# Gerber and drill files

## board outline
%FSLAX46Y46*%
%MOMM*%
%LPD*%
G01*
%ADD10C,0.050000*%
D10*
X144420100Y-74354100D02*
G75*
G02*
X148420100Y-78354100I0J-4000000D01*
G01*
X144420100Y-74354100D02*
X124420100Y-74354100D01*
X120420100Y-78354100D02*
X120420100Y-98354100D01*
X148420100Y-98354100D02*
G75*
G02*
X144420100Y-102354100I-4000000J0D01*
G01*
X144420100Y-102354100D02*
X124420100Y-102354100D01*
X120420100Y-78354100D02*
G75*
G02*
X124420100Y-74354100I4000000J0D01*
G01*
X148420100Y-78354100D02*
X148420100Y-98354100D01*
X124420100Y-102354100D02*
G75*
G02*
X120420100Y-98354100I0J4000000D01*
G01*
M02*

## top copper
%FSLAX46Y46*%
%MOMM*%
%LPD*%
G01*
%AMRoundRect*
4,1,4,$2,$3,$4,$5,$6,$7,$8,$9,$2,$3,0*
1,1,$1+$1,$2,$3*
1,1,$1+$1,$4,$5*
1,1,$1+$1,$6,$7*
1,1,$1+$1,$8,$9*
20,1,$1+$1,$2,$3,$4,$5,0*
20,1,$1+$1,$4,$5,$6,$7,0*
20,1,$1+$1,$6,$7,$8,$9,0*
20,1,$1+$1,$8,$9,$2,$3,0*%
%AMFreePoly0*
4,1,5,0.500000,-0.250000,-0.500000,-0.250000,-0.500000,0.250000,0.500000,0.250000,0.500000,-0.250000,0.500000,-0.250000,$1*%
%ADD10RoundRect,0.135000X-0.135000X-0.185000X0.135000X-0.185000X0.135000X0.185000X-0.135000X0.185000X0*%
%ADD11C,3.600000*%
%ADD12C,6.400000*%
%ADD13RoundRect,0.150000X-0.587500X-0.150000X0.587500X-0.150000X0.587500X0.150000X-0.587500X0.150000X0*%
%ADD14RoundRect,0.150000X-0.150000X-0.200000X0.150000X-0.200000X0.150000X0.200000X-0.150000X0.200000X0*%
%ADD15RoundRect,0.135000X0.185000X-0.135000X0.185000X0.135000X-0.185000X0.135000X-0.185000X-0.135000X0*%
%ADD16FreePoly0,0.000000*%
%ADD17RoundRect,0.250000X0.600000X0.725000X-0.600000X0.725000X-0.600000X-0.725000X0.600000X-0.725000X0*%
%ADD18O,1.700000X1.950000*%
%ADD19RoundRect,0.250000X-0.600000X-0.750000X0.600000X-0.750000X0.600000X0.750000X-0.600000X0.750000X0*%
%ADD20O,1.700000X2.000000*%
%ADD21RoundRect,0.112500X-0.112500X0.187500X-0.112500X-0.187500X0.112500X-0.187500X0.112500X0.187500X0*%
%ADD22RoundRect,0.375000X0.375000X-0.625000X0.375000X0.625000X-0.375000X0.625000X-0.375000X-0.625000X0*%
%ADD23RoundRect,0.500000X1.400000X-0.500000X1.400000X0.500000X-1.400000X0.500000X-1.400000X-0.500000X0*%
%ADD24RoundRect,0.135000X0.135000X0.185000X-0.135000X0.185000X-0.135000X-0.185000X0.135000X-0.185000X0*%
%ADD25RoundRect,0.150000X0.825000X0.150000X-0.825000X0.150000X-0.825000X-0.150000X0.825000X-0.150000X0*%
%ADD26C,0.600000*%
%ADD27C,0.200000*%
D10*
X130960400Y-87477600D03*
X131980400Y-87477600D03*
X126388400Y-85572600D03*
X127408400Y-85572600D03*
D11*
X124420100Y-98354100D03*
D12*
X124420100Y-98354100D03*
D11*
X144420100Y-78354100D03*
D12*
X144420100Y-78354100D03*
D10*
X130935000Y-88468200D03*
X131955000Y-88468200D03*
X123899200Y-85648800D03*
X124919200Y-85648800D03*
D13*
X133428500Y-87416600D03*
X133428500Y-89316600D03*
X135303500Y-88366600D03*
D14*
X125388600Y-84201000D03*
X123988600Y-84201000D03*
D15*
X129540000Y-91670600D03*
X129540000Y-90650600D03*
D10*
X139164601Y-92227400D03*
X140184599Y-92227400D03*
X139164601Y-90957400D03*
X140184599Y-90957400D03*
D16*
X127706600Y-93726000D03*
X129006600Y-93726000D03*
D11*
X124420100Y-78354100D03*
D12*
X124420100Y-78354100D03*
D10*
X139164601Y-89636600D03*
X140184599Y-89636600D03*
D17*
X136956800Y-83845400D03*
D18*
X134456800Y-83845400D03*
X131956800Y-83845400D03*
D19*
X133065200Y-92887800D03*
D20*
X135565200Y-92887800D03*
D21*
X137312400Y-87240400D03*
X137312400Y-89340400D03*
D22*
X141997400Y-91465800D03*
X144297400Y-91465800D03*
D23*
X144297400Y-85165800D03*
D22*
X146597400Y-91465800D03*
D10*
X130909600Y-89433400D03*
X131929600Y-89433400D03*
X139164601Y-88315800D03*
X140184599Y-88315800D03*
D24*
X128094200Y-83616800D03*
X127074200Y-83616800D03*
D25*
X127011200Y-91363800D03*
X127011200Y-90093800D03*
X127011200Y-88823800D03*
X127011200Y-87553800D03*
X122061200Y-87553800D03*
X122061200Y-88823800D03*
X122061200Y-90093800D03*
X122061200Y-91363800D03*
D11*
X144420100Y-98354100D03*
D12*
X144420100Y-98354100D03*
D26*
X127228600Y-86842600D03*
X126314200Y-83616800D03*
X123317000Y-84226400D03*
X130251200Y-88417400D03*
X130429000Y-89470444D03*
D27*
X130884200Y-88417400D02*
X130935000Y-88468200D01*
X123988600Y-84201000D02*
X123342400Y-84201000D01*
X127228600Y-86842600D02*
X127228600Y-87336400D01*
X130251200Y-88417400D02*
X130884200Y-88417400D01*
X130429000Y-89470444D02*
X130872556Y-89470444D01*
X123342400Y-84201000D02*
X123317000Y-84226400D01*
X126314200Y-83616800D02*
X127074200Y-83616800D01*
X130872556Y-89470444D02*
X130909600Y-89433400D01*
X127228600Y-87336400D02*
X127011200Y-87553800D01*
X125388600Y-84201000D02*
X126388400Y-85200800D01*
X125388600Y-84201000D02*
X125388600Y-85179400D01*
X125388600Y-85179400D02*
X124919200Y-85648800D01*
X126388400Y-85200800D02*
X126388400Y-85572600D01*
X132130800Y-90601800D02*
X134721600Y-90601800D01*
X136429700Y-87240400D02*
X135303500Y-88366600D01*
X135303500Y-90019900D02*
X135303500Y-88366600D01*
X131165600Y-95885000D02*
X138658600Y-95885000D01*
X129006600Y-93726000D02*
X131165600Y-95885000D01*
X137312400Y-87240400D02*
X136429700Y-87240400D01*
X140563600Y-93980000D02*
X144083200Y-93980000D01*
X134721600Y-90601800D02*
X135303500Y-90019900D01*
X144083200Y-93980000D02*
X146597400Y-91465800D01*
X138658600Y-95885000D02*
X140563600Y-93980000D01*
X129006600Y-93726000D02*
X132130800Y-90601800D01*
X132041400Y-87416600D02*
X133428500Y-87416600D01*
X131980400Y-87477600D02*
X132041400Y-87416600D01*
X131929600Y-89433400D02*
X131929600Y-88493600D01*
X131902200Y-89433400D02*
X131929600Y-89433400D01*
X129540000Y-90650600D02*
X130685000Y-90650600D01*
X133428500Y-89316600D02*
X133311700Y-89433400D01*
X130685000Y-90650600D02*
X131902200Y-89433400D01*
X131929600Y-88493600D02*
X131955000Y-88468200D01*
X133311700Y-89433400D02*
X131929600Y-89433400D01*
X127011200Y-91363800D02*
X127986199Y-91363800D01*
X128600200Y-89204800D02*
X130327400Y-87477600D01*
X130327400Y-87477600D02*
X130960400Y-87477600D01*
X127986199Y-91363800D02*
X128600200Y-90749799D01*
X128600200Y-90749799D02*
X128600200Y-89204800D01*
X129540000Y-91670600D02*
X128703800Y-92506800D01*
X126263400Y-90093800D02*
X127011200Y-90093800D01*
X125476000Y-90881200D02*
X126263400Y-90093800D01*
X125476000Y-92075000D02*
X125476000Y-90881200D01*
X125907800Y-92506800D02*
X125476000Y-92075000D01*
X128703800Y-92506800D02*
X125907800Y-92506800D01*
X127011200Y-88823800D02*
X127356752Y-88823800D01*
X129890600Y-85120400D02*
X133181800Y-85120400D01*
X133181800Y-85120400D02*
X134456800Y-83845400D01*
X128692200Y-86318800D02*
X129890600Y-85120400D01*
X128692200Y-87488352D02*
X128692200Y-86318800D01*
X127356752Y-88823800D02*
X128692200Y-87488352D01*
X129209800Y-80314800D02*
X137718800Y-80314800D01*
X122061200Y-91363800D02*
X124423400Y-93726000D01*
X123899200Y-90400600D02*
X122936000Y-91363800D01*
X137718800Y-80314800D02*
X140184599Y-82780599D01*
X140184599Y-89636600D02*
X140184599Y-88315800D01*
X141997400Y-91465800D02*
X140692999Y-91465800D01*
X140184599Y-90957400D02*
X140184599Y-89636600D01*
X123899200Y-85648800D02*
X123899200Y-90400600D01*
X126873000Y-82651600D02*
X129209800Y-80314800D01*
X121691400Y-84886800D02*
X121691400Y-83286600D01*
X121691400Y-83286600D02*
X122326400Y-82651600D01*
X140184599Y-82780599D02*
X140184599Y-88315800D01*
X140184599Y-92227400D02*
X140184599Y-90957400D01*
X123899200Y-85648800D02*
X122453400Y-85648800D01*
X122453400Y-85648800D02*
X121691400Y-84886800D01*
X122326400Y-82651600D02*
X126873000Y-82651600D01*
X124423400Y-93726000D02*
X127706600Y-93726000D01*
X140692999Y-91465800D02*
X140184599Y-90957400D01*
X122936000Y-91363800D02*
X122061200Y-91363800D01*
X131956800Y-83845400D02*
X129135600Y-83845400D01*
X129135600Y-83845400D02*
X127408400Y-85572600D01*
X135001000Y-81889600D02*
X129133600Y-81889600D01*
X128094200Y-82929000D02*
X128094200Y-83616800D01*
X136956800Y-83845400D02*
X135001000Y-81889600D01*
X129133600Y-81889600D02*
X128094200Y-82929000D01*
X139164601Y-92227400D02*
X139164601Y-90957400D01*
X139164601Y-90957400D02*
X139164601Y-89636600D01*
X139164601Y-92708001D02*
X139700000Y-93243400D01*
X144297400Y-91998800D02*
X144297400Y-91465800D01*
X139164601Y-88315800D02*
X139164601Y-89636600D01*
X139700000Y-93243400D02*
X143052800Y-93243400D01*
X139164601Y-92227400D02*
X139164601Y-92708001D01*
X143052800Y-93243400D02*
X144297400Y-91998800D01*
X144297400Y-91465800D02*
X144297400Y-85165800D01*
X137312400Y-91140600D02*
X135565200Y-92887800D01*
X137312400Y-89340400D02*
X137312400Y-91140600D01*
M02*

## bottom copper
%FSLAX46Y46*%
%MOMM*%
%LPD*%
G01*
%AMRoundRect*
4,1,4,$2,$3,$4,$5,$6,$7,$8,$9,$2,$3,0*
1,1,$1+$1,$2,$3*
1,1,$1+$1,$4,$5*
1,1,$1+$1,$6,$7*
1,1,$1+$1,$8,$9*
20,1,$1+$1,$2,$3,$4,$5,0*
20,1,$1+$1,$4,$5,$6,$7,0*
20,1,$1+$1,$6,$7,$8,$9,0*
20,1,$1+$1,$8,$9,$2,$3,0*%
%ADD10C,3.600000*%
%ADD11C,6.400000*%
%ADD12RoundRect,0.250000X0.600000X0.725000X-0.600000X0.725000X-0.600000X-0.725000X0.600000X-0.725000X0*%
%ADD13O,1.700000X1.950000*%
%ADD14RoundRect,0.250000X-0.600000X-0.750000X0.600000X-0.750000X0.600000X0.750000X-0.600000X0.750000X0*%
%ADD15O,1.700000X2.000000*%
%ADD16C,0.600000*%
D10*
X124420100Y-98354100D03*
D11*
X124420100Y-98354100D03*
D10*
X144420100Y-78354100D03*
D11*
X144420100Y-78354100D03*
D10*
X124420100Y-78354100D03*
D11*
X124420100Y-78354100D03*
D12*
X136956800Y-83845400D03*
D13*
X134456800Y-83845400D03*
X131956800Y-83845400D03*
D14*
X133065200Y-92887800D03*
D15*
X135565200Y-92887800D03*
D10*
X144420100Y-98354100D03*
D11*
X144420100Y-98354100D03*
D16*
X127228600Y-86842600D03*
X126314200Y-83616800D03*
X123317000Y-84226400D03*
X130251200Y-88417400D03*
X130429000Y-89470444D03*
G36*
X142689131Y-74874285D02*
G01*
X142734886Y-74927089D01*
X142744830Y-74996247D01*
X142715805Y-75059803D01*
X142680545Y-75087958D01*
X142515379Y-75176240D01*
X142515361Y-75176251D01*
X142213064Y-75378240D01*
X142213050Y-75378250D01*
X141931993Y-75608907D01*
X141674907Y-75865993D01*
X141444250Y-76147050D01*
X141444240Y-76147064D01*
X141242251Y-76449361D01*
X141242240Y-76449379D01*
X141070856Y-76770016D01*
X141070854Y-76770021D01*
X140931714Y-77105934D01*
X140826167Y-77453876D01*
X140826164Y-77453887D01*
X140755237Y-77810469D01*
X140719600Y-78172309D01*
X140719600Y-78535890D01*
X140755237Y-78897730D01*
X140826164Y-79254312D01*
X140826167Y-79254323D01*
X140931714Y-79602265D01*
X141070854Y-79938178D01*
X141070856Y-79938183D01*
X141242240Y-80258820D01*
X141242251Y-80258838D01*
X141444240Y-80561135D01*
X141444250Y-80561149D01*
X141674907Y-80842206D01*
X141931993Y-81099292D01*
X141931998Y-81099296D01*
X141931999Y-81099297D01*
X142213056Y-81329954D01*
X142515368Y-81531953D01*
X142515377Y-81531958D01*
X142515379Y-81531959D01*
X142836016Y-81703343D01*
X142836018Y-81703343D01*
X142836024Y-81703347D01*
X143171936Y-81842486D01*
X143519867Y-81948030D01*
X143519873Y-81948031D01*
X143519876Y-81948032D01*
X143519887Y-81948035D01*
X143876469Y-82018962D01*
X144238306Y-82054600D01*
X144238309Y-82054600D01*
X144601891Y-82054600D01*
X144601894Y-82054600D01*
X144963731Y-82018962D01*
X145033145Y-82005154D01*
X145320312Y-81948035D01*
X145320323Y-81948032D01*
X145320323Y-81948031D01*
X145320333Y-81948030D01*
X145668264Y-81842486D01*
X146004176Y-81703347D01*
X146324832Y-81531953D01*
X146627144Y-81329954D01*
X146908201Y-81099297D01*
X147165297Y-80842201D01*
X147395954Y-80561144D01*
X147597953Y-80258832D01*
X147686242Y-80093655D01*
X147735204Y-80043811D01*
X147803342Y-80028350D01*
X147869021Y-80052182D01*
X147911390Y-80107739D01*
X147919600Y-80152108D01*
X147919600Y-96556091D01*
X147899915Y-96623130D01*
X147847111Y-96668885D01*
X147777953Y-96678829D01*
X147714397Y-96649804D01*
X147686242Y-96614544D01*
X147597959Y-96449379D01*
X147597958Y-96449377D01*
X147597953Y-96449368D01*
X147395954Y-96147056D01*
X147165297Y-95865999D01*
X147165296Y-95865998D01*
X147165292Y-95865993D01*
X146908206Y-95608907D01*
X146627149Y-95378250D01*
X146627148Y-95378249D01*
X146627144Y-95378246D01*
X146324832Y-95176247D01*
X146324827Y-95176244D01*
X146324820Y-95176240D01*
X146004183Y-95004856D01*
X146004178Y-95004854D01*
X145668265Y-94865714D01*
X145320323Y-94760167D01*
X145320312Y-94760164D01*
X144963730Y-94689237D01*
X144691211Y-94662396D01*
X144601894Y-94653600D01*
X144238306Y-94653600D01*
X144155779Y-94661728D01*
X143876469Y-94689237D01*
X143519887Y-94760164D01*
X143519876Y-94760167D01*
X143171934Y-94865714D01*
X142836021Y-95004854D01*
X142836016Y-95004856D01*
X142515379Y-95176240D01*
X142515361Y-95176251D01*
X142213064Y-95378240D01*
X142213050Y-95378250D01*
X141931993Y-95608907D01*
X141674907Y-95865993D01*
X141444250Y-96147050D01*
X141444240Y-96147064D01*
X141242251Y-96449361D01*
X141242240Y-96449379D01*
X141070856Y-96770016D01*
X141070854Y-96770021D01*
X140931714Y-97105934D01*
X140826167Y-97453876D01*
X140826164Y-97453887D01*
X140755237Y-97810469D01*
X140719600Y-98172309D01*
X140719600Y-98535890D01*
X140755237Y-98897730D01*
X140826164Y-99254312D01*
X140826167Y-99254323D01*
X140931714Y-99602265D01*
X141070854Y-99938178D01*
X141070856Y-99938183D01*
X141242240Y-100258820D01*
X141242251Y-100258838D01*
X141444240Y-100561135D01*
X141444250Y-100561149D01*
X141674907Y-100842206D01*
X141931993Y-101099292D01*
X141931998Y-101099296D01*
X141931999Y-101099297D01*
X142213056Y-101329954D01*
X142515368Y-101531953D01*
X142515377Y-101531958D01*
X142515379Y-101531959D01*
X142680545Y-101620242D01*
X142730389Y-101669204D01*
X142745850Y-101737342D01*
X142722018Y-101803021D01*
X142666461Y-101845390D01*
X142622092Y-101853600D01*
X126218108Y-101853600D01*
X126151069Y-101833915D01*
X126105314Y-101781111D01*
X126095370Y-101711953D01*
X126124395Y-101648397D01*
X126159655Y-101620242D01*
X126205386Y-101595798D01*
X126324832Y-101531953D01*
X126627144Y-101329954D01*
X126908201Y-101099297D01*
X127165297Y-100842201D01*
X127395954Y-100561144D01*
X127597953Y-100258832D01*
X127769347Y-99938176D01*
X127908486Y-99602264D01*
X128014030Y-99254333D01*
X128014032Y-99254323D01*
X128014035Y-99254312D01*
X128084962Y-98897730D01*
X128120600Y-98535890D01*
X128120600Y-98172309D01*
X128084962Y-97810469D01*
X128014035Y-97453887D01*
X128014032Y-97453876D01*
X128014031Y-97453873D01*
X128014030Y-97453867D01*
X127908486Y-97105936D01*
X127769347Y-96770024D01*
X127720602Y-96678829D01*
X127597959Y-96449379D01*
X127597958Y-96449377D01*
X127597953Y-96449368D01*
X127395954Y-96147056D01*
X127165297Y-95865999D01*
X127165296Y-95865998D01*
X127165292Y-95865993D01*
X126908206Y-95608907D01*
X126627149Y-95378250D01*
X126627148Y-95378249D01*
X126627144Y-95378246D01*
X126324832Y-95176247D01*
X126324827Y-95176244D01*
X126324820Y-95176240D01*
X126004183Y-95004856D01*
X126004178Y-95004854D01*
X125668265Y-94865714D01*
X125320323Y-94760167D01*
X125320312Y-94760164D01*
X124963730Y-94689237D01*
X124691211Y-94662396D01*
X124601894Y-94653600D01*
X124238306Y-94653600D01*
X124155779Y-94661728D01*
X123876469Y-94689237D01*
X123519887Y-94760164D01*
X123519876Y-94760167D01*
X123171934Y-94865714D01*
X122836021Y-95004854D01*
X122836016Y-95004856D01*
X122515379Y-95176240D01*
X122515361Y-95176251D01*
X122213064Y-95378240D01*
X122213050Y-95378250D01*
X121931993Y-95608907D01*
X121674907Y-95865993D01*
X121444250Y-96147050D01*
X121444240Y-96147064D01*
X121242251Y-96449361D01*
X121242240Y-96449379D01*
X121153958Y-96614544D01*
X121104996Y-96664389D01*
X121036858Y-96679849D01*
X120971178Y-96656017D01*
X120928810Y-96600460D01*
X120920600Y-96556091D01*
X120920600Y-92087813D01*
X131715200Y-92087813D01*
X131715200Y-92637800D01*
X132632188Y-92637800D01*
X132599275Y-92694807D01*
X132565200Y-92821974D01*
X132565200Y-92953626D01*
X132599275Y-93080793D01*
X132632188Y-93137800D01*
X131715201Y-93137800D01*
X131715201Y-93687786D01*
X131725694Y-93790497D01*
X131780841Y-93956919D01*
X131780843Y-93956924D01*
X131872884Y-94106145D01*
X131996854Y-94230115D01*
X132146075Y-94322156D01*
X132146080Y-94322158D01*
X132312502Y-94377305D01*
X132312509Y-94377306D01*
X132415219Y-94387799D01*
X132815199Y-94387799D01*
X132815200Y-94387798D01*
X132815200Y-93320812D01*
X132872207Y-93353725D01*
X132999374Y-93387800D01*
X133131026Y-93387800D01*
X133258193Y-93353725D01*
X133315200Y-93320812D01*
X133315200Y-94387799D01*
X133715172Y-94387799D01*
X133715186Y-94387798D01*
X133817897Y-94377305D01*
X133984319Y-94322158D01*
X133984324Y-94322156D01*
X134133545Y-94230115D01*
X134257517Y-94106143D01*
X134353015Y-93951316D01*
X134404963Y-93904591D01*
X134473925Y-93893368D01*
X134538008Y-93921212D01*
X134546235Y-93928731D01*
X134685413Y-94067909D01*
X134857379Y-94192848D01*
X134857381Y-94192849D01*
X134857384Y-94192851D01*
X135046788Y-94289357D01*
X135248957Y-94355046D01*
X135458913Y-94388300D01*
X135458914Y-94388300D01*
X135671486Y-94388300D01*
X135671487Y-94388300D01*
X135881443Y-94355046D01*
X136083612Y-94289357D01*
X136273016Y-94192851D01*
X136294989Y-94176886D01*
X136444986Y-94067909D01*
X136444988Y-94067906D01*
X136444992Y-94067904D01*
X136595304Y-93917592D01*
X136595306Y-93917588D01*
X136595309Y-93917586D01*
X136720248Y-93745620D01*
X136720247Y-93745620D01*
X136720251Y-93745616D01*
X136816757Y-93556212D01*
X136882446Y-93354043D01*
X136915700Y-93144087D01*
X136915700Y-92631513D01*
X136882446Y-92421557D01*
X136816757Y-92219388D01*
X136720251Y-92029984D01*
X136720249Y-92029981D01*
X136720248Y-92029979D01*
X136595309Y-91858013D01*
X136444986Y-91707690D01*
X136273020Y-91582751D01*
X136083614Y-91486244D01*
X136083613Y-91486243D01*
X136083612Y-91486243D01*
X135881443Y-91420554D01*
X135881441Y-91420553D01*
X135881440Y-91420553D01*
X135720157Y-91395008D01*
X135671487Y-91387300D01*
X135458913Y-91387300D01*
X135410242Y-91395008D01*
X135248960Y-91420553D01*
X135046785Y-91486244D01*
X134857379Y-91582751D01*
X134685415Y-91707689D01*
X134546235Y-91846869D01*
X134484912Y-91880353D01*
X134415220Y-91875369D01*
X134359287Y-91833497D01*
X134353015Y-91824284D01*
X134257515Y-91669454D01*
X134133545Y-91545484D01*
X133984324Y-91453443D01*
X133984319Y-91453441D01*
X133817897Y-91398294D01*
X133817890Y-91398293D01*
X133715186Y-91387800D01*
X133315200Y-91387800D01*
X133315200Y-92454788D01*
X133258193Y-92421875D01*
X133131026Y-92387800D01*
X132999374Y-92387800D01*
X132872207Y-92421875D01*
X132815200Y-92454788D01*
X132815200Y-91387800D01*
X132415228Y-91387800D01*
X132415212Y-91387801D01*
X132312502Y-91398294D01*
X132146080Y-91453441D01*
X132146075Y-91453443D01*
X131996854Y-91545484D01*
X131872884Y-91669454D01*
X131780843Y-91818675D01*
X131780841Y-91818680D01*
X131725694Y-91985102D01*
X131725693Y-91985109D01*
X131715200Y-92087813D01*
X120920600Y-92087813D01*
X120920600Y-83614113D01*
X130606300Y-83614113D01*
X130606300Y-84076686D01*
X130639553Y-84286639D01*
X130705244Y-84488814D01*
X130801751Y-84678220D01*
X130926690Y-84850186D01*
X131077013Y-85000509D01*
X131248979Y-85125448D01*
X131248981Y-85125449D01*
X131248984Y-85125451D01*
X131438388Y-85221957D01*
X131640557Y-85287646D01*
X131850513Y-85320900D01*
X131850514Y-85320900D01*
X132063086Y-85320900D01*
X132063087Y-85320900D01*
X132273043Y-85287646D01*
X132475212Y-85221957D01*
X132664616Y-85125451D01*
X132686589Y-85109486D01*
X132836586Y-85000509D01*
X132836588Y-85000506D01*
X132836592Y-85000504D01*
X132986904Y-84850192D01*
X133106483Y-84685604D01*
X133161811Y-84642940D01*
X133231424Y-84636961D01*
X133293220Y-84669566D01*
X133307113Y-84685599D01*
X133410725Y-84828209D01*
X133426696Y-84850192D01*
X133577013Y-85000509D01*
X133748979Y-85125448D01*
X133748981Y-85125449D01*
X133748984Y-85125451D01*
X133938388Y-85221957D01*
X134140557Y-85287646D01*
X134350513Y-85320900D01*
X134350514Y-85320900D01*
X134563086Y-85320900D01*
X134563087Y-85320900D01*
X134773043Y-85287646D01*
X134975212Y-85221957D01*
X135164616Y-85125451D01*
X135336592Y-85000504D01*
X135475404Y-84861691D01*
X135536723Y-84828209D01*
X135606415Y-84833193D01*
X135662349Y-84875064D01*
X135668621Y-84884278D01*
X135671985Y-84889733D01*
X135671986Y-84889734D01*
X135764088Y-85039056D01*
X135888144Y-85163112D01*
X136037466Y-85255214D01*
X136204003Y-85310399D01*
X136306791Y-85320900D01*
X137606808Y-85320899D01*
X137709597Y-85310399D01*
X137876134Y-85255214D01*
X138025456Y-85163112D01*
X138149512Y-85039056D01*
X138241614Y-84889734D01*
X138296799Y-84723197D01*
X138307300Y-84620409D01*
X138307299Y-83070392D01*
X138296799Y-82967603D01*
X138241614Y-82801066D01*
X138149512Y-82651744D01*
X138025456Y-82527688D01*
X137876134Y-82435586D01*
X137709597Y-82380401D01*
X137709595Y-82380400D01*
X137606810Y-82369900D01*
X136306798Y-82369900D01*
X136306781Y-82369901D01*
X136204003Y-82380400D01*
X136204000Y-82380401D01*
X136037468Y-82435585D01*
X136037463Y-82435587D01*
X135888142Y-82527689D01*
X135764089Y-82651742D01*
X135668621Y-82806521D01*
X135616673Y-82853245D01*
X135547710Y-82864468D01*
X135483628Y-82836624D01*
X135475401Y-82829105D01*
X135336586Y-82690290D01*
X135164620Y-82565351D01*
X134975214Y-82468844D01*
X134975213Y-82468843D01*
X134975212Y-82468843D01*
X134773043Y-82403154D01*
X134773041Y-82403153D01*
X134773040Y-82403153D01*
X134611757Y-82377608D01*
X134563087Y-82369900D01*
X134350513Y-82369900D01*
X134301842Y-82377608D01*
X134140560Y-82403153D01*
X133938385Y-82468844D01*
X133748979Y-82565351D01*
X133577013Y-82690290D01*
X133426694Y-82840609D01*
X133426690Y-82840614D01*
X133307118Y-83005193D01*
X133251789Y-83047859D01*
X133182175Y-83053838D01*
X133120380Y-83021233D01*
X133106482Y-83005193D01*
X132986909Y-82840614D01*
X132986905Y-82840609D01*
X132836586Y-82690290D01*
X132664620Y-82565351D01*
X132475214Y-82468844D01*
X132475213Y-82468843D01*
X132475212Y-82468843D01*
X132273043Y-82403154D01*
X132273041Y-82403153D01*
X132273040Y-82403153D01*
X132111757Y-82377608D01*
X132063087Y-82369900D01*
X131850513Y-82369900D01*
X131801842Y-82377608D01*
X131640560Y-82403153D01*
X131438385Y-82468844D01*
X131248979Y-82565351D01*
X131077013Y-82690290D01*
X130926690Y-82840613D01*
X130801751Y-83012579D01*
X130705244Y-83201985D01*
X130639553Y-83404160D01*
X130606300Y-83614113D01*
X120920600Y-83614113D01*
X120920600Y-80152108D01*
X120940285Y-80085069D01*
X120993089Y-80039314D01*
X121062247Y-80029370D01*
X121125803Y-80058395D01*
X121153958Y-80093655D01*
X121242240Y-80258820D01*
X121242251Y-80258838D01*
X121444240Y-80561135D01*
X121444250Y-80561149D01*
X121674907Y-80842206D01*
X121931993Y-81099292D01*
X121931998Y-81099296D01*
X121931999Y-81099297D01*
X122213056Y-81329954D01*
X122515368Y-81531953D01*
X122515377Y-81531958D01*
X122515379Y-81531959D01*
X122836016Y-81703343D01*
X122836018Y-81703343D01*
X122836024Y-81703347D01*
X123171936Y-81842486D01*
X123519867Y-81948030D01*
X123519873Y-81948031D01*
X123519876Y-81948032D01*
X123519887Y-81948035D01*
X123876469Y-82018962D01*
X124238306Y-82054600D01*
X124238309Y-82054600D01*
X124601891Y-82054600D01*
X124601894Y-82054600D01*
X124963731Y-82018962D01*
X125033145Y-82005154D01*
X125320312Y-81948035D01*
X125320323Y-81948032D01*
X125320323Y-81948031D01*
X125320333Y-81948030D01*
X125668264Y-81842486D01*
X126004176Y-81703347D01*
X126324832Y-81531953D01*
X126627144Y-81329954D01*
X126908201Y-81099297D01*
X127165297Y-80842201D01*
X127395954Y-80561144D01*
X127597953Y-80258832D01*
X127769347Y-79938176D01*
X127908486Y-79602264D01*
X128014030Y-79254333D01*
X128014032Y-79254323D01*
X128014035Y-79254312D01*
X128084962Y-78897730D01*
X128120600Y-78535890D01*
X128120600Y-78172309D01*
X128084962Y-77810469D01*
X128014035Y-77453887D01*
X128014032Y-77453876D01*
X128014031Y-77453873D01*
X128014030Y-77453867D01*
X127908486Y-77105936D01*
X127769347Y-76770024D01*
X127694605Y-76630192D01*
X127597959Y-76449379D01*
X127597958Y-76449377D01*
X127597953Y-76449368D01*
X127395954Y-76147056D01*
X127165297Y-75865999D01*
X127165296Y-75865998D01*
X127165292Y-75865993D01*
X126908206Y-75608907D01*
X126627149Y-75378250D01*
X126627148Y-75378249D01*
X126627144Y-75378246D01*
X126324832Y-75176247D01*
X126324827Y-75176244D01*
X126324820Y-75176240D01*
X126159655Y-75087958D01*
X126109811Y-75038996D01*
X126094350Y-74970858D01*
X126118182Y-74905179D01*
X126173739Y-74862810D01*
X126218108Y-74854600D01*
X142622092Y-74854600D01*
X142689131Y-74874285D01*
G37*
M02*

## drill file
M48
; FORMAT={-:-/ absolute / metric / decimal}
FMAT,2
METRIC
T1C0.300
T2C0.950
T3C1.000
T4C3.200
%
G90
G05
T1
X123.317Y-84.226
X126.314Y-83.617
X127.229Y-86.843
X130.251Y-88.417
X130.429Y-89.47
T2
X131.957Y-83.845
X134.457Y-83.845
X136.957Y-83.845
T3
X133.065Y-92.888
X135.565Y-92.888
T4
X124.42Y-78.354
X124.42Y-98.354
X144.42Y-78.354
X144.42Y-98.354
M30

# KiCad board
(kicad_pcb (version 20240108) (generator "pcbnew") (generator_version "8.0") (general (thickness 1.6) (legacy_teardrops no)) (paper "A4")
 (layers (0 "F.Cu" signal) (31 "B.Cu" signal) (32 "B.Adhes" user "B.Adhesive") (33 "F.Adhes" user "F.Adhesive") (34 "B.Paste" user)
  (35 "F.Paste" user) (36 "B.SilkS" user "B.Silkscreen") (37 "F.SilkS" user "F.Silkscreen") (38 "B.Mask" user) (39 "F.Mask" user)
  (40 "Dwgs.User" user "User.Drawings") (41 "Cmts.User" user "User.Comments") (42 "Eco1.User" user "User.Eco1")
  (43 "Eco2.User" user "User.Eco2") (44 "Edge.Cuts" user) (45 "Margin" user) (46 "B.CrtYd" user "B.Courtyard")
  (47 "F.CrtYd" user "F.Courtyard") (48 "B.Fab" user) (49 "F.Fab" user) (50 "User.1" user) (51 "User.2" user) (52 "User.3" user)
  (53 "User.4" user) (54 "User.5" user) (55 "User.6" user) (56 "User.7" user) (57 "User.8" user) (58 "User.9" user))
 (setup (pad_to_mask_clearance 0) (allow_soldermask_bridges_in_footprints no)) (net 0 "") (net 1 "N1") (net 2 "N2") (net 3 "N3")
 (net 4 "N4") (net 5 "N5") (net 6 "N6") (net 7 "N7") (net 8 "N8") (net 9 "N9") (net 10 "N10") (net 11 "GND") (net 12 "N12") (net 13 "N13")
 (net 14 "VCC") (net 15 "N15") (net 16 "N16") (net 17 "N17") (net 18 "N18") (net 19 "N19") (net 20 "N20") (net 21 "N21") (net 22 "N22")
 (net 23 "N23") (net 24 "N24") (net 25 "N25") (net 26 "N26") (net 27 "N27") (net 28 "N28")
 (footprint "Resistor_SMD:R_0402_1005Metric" (layer "F.Cu") (at 131.4704 87.4776)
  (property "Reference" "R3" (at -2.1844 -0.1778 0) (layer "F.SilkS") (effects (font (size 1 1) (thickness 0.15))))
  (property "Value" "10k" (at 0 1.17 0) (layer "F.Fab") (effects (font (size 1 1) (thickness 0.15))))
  (pad "1" smd roundrect (at -0.51 0) (size 0.54 0.64) (layers "F.Cu" "F.Paste" "F.Mask") (roundrect_rratio 0.25) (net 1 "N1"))
  (pad "2" smd roundrect (at 0.51 0) (size 0.54 0.64) (layers "F.Cu" "F.Paste" "F.Mask") (roundrect_rratio 0.25) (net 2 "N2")))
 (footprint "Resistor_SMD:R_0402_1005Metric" (layer "F.Cu") (at 126.8984 85.5726)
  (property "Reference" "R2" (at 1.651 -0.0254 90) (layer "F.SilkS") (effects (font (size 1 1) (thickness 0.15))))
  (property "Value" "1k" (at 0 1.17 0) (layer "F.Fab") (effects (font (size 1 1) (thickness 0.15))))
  (pad "1" smd roundrect (at -0.51 0) (size 0.54 0.64) (layers "F.Cu" "F.Paste" "F.Mask") (roundrect_rratio 0.25) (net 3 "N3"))
  (pad "2" smd roundrect (at 0.51 0) (size 0.54 0.64) (layers "F.Cu" "F.Paste" "F.Mask") (roundrect_rratio 0.25) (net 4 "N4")))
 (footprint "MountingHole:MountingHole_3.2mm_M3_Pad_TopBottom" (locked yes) (layer "F.Cu") (at 124.4201 98.3541)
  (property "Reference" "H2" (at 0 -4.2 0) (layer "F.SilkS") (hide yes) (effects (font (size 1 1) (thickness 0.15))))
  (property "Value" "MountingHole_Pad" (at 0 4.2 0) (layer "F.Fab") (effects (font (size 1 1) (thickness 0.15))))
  (pad "1" thru_hole circle (at 0 0) (size 3.6 3.6) (drill 3.2) (layers "*.Cu" "*.Mask") (remove_unused_layers no) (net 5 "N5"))
  (pad "1" connect circle (at 0 0) (size 6.4 6.4) (layers "F.Cu" "F.Mask") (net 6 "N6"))
  (pad "1" connect circle (at 0 0) (size 6.4 6.4) (layers "B.Cu" "B.Mask") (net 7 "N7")))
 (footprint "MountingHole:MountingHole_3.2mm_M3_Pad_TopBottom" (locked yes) (layer "F.Cu") (at 144.4201 78.3541)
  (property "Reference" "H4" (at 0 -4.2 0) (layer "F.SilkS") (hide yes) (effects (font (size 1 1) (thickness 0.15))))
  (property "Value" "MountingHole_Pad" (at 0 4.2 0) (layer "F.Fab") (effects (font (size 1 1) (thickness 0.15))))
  (pad "1" thru_hole circle (at 0 0) (size 3.6 3.6) (drill 3.2) (layers "*.Cu" "*.Mask") (remove_unused_layers no) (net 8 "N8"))
  (pad "1" connect circle (at 0 0) (size 6.4 6.4) (layers "F.Cu" "F.Mask") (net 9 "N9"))
  (pad "1" connect circle (at 0 0) (size 6.4 6.4) (layers "B.Cu" "B.Mask") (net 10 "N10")))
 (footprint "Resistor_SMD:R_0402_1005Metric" (layer "F.Cu") (at 131.445 88.4682)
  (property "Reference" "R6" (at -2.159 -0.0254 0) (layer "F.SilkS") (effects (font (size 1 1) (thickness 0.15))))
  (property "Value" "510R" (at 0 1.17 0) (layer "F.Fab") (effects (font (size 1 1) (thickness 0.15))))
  (pad "1" smd roundrect (at -0.51 0) (size 0.54 0.64) (layers "F.Cu" "F.Paste" "F.Mask") (roundrect_rratio 0.25) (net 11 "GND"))
  (pad "2" smd roundrect (at 0.51 0) (size 0.54 0.64) (layers "F.Cu" "F.Paste" "F.Mask") (roundrect_rratio 0.25) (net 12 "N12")))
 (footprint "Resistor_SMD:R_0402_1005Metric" (layer "F.Cu") (at 124.4092 85.6488)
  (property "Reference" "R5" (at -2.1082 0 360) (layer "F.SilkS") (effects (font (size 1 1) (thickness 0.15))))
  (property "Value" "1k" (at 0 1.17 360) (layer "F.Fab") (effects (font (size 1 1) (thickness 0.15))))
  (pad "1" smd roundrect (at -0.51 0) (size 0.54 0.64) (layers "F.Cu" "F.Paste" "F.Mask") (roundrect_rratio 0.25) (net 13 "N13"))
  (pad "2" smd roundrect (at 0.51 0) (size 0.54 0.64) (layers "F.Cu" "F.Paste" "F.Mask") (roundrect_rratio 0.25) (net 3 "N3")))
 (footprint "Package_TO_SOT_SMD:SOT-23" (layer "F.Cu") (at 134.366 88.3666)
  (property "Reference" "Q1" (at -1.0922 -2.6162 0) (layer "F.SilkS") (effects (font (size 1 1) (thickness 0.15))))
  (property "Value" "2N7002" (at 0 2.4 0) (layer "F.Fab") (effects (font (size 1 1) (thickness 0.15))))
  (pad "1" smd roundrect (at -0.9375 -0.95) (size 1.475 0.6) (layers "F.Cu" "F.Paste" "F.Mask") (roundrect_rratio 0.25) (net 2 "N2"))
  (pad "2" smd roundrect (at -0.9375 0.95) (size 1.475 0.6) (layers "F.Cu" "F.Paste" "F.Mask") (roundrect_rratio 0.25) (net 12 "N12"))
  (pad "3" smd roundrect (at 0.9375 0) (size 1.475 0.6) (layers "F.Cu" "F.Paste" "F.Mask") (roundrect_rratio 0.25) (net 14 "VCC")))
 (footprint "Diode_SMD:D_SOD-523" (layer "F.Cu") (at 124.6886 84.201 180)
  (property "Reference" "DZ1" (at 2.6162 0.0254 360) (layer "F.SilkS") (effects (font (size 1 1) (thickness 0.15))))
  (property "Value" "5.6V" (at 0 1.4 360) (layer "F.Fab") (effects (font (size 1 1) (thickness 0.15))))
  (pad "1" smd roundrect (at -0.7 0) (size 0.6 0.7) (layers "F.Cu" "F.Paste" "F.Mask") (roundrect_rratio 0.25) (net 3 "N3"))
  (pad "2" smd roundrect (at 0.7 0) (size 0.6 0.7) (layers "F.Cu" "F.Paste" "F.Mask") (roundrect_rratio 0.25) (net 11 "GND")))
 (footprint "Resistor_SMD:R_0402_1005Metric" (layer "F.Cu") (at 129.54 91.1606 90)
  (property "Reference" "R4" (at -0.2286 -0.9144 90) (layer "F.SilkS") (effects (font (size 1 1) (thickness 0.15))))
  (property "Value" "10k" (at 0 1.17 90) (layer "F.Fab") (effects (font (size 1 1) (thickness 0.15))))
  (pad "1" smd roundrect (at -0.51 0 90) (size 0.54 0.64) (layers "F.Cu" "F.Paste" "F.Mask") (roundrect_rratio 0.25) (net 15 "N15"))
  (pad "2" smd roundrect (at 0.51 0 90) (size 0.54 0.64) (layers "F.Cu" "F.Paste" "F.Mask") (roundrect_rratio 0.25) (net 12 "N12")))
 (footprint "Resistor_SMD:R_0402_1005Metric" (layer "F.Cu") (at 139.6746 92.2274)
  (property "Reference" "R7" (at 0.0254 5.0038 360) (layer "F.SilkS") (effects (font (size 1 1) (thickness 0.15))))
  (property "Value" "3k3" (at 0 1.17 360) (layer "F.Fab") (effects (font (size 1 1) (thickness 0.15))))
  (pad "1" smd roundrect (at -0.509999 0) (size 0.54 0.64) (layers "F.Cu" "F.Paste" "F.Mask") (roundrect_rratio 0.25) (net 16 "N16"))
  (pad "2" smd roundrect (at 0.509999 0) (size 0.54 0.64) (layers "F.Cu" "F.Paste" "F.Mask") (roundrect_rratio 0.25) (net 13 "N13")))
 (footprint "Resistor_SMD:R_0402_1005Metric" (layer "F.Cu") (at 139.6746 90.9574)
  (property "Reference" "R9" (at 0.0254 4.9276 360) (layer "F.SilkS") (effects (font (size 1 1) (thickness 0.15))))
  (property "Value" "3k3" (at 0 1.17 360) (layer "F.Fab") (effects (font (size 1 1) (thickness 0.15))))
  (pad "1" smd roundrect (at -0.509999 0) (size 0.54 0.64) (layers "F.Cu" "F.Paste" "F.Mask") (roundrect_rratio 0.25) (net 16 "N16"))
  (pad "2" smd roundrect (at 0.509999 0) (size 0.54 0.64) (layers "F.Cu" "F.Paste" "F.Mask") (roundrect_rratio 0.25) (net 13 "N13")))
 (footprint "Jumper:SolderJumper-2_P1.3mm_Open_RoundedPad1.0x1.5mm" (layer "F.Cu") (at 128.3566 93.726)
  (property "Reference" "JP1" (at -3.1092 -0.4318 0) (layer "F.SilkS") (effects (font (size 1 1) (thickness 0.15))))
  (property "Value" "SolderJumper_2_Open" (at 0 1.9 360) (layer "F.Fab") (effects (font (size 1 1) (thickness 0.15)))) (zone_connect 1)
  (pad "1" smd custom (at -0.65 0) (size 1 0.5) (layers "F.Cu" "F.Mask") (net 13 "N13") (zone_connect 2) (thermal_bridge_angle 45)
   (options (clearance outline) (anchor rect)) (primitives))
  (pad "2" smd custom (at 0.65 0) (size 1 0.5) (layers "F.Cu" "F.Mask") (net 14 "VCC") (zone_connect 2) (thermal_bridge_angle 45)
   (options (clearance outline) (anchor rect)) (primitives)))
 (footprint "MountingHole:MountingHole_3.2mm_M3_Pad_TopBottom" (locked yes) (layer "F.Cu") (at 124.4201 78.3541)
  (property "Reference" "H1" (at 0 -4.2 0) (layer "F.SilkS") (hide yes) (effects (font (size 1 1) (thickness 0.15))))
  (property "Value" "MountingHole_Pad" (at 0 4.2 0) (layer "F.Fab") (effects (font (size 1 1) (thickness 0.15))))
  (pad "1" thru_hole circle (at 0 0) (size 3.6 3.6) (drill 3.2) (layers "*.Cu" "*.Mask") (remove_unused_layers no) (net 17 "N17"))
  (pad "1" connect circle (at 0 0) (size 6.4 6.4) (layers "F.Cu" "F.Mask") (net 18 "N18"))
  (pad "1" connect circle (at 0 0) (size 6.4 6.4) (layers "B.Cu" "B.Mask") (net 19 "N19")))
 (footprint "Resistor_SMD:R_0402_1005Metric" (layer "F.Cu") (at 139.6746 89.6366)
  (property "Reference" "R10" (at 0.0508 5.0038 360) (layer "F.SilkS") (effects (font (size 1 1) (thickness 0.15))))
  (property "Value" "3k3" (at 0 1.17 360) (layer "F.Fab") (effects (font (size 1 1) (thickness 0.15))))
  (pad "1" smd roundrect (at -0.509999 0) (size 0.54 0.64) (layers "F.Cu" "F.Paste" "F.Mask") (roundrect_rratio 0.25) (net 16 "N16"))
  (pad "2" smd roundrect (at 0.509999 0) (size 0.54 0.64) (layers "F.Cu" "F.Paste" "F.Mask") (roundrect_rratio 0.25) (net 13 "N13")))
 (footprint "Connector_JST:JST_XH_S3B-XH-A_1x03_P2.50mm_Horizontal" (layer "F.Cu") (at 136.9568 83.8454 180)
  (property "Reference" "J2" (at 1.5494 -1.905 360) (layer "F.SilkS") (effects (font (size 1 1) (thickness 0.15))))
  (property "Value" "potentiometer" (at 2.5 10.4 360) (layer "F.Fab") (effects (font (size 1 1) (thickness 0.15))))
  (pad "1" thru_hole roundrect (at 0 0 180) (size 1.7 1.95) (drill 0.95) (layers "*.Cu" "*.Mask") (remove_unused_layers no)
   (roundrect_rratio 0.147059) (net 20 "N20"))
  (pad "2" thru_hole oval (at 2.5 0 180) (size 1.7 1.95) (drill 0.95) (layers "*.Cu" "*.Mask") (remove_unused_layers no) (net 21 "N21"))
  (pad "3" thru_hole oval (at 5 0 180) (size 1.7 1.95) (drill 0.95) (layers "*.Cu" "*.Mask") (remove_unused_layers no) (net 4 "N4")))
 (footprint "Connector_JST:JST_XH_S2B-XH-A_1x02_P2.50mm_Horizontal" (layer "F.Cu") (at 133.0652 92.8878)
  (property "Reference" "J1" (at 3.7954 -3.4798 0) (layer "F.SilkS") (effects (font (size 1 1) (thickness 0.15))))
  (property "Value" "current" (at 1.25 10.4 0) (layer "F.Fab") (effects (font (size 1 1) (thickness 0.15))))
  (pad "1" thru_hole roundrect (at 0 0) (size 1.7 2) (drill 1) (layers "*.Cu" "*.Mask") (remove_unused_layers no)
   (roundrect_rratio 0.147059) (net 11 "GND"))
  (pad "2" thru_hole oval (at 2.5 0) (size 1.7 2) (drill 1) (layers "*.Cu" "*.Mask") (remove_unused_layers no) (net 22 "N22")))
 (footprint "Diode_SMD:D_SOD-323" (layer "F.Cu") (at 137.3124 88.2904 -90)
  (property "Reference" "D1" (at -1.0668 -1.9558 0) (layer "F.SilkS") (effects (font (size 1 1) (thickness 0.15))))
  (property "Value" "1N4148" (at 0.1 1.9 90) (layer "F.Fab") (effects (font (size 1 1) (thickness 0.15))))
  (pad "1" smd roundrect (at -1.05 0 270) (size 0.6 0.45) (layers "F.Cu" "F.Paste" "F.Mask") (roundrect_rratio 0.25) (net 14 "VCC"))
  (pad "2" smd roundrect (at 1.05 0 270) (size 0.6 0.45) (layers "F.Cu" "F.Paste" "F.Mask") (roundrect_rratio 0.25) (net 22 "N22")))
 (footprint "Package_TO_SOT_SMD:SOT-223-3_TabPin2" (layer "F.Cu") (at 144.2974 88.3158 90)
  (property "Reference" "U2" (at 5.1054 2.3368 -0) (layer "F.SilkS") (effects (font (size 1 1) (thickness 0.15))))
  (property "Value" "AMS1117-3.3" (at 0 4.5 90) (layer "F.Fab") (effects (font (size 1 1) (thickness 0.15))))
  (pad "1" smd roundrect (at -3.15 -2.3 90) (size 2 1.5) (layers "F.Cu" "F.Paste" "F.Mask") (roundrect_rratio 0.25) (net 13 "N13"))
  (pad "2" smd roundrect (at -3.15 0 90) (size 2 1.5) (layers "F.Cu" "F.Paste" "F.Mask") (roundrect_rratio 0.25) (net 16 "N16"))
  (pad "2" smd roundrect (at 3.15 0 90) (size 2 3.8) (layers "F.Cu" "F.Paste" "F.Mask") (roundrect_rratio 0.25) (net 16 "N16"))
  (pad "3" smd roundrect (at -3.15 2.3 90) (size 2 1.5) (layers "F.Cu" "F.Paste" "F.Mask") (roundrect_rratio 0.25) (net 14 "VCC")))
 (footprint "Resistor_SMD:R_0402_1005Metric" (layer "F.Cu") (at 131.4196 89.4334)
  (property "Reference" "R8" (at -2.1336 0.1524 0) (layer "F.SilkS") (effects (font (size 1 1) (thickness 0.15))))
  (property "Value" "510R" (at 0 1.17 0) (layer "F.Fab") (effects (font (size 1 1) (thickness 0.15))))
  (pad "1" smd roundrect (at -0.51 0) (size 0.54 0.64) (layers "F.Cu" "F.Paste" "F.Mask") (roundrect_rratio 0.25) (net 11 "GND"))
  (pad "2" smd roundrect (at 0.51 0) (size 0.54 0.64) (layers "F.Cu" "F.Paste" "F.Mask") (roundrect_rratio 0.25) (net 12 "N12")))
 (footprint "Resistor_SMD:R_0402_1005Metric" (layer "F.Cu") (at 139.6746 88.3158)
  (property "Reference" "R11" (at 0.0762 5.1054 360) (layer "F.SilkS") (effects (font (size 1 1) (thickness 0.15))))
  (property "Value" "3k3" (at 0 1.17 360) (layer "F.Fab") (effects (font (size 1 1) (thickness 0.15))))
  (pad "1" smd roundrect (at -0.509999 0) (size 0.54 0.64) (layers "F.Cu" "F.Paste" "F.Mask") (roundrect_rratio 0.25) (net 16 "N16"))
  (pad "2" smd roundrect (at 0.509999 0) (size 0.54 0.64) (layers "F.Cu" "F.Paste" "F.Mask") (roundrect_rratio 0.25) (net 13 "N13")))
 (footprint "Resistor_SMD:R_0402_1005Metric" (layer "F.Cu") (at 127.5842 83.6168 180)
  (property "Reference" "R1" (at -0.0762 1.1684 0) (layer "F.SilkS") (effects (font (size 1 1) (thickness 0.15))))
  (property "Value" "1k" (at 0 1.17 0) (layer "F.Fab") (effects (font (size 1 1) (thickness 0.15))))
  (pad "1" smd roundrect (at -0.51 0 180) (size 0.54 0.64) (layers "F.Cu" "F.Paste" "F.Mask") (roundrect_rratio 0.25) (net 20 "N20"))
  (pad "2" smd roundrect (at 0.51 0 180) (size 0.54 0.64) (layers "F.Cu" "F.Paste" "F.Mask") (roundrect_rratio 0.25) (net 11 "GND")))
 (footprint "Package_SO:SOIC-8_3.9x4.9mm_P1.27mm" (layer "F.Cu") (at 124.5362 89.4588 180)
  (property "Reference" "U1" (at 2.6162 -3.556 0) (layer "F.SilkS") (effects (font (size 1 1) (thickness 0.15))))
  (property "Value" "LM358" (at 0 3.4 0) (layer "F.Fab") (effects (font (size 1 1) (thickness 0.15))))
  (pad "1" smd roundrect (at -2.475 -1.905 180) (size 1.95 0.6) (layers "F.Cu" "F.Paste" "F.Mask") (roundrect_rratio 0.25) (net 1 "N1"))
  (pad "2" smd roundrect (at -2.475 -0.635 180) (size 1.95 0.6) (layers "F.Cu" "F.Paste" "F.Mask") (roundrect_rratio 0.25) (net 15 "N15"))
  (pad "3" smd roundrect (at -2.475 0.635 180) (size 1.95 0.6) (layers "F.Cu" "F.Paste" "F.Mask") (roundrect_rratio 0.25) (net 21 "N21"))
  (pad "4" smd roundrect (at -2.475 1.905 180) (size 1.95 0.6) (layers "F.Cu" "F.Paste" "F.Mask") (roundrect_rratio 0.25) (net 11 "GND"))
  (pad "5" smd roundrect (at 2.475 1.905 180) (size 1.95 0.6) (layers "F.Cu" "F.Paste" "F.Mask") (roundrect_rratio 0.25) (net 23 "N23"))
  (pad "6" smd roundrect (at 2.475 0.635 180) (size 1.95 0.6) (layers "F.Cu" "F.Paste" "F.Mask") (roundrect_rratio 0.25) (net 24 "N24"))
  (pad "7" smd roundrect (at 2.475 -0.635 180) (size 1.95 0.6) (layers "F.Cu" "F.Paste" "F.Mask") (roundrect_rratio 0.25) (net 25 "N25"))
  (pad "8" smd roundrect (at 2.475 -1.905 180) (size 1.95 0.6) (layers "F.Cu" "F.Paste" "F.Mask") (roundrect_rratio 0.25) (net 13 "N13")))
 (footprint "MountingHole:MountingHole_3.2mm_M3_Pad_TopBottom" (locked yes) (layer "F.Cu") (at 144.4201 98.3541)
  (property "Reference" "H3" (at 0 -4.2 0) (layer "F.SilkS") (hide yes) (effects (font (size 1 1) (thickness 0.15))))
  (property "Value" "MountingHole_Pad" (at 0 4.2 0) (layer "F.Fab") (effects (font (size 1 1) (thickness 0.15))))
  (pad "1" thru_hole circle (at 0 0) (size 3.6 3.6) (drill 3.2) (layers "*.Cu" "*.Mask") (remove_unused_layers no) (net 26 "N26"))
  (pad "1" connect circle (at 0 0) (size 6.4 6.4) (layers "F.Cu" "F.Mask") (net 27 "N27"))
  (pad "1" connect circle (at 0 0) (size 6.4 6.4) (layers "B.Cu" "B.Mask") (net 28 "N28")))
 (gr_arc (start 144.4201 74.3541) (mid 147.248527 75.525673) (end 148.4201 78.3541) (stroke (width 0.05) (type default)) (layer "Edge.Cuts"))
 (gr_line (start 144.4201 74.3541) (end 124.4201 74.3541) (stroke (width 0.05) (type default)) (layer "Edge.Cuts"))
 (gr_line (start 120.4201 78.3541) (end 120.4201 98.3541) (stroke (width 0.05) (type default)) (layer "Edge.Cuts"))
 (gr_arc (start 148.4201 98.3541) (mid 147.248527 101.182527) (end 144.4201 102.3541) (stroke (width 0.05) (type default))
  (layer "Edge.Cuts"))
 (gr_line (start 144.4201 102.3541) (end 124.4201 102.3541) (stroke (width 0.05) (type default)) (layer "Edge.Cuts"))
 (gr_arc (start 120.4201 78.3541) (mid 121.591673 75.525673) (end 124.4201 74.3541) (stroke (width 0.05) (type default)) (layer "Edge.Cuts"))
 (gr_line (start 148.4201 78.3541) (end 148.4201 98.3541) (stroke (width 0.05) (type default)) (layer "Edge.Cuts"))
 (gr_arc (start 124.4201 102.3541) (mid 121.591673 101.182527) (end 120.4201 98.3541) (stroke (width 0.05) (type default))
  (layer "Edge.Cuts"))
 (segment (start 130.8842 88.4174) (end 130.935 88.4682) (width 0.2) (layer "F.Cu") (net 11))
 (segment (start 123.9886 84.201) (end 123.3424 84.201) (width 0.2) (layer "F.Cu") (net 11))
 (segment (start 127.2286 86.8426) (end 127.2286 87.3364) (width 0.2) (layer "F.Cu") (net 11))
 (segment (start 130.2512 88.4174) (end 130.8842 88.4174) (width 0.2) (layer "F.Cu") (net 11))
 (segment (start 130.429 89.470444) (end 130.872556 89.470444) (width 0.2) (layer "F.Cu") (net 11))
 (segment (start 123.3424 84.201) (end 123.317 84.2264) (width 0.2) (layer "F.Cu") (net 11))
 (segment (start 126.3142 83.6168) (end 127.0742 83.6168) (width 0.2) (layer "F.Cu") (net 11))
 (segment (start 130.872556 89.470444) (end 130.9096 89.4334) (width 0.2) (layer "F.Cu") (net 11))
 (segment (start 127.2286 87.3364) (end 127.0112 87.5538) (width 0.2) (layer "F.Cu") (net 11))
 (via (at 127.2286 86.8426) (size 0.6) (drill 0.3) (layers "F.Cu" "B.Cu") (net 11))
 (via (at 126.3142 83.6168) (size 0.6) (drill 0.3) (layers "F.Cu" "B.Cu") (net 11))
 (via (at 123.317 84.2264) (size 0.6) (drill 0.3) (layers "F.Cu" "B.Cu") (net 11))
 (via (at 130.2512 88.4174) (size 0.6) (drill 0.3) (layers "F.Cu" "B.Cu") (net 11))
 (via (at 130.429 89.470444) (size 0.6) (drill 0.3) (layers "F.Cu" "B.Cu") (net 11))
 (segment (start 125.3886 84.201) (end 126.3884 85.2008) (width 0.2) (layer "F.Cu") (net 3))
 (segment (start 125.3886 84.201) (end 125.3886 85.1794) (width 0.2) (layer "F.Cu") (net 3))
 (segment (start 125.3886 85.1794) (end 124.9192 85.6488) (width 0.2) (layer "F.Cu") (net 3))
 (segment (start 126.3884 85.2008) (end 126.3884 85.5726) (width 0.2) (layer "F.Cu") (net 3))
 (segment (start 132.1308 90.6018) (end 134.7216 90.6018) (width 0.2) (layer "F.Cu") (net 14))
 (segment (start 136.4297 87.2404) (end 135.3035 88.3666) (width 0.2) (layer "F.Cu") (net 14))
 (segment (start 135.3035 90.0199) (end 135.3035 88.3666) (width 0.2) (layer "F.Cu") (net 14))
 (segment (start 131.1656 95.885) (end 138.6586 95.885) (width 0.2) (layer "F.Cu") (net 14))
 (segment (start 129.0066 93.726) (end 131.1656 95.885) (width 0.2) (layer "F.Cu") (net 14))
 (segment (start 137.3124 87.2404) (end 136.4297 87.2404) (width 0.2) (layer "F.Cu") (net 14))
 (segment (start 140.5636 93.98) (end 144.0832 93.98) (width 0.2) (layer "F.Cu") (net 14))
 (segment (start 134.7216 90.6018) (end 135.3035 90.0199) (width 0.2) (layer "F.Cu") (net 14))
 (segment (start 144.0832 93.98) (end 146.5974 91.4658) (width 0.2) (layer "F.Cu") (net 14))
 (segment (start 138.6586 95.885) (end 140.5636 93.98) (width 0.2) (layer "F.Cu") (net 14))
 (segment (start 129.0066 93.726) (end 132.1308 90.6018) (width 0.2) (layer "F.Cu") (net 14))
 (segment (start 132.0414 87.4166) (end 133.4285 87.4166) (width 0.2) (layer "F.Cu") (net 2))
 (segment (start 131.9804 87.4776) (end 132.0414 87.4166) (width 0.2) (layer "F.Cu") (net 2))
 (segment (start 131.9296 89.4334) (end 131.9296 88.4936) (width 0.2) (layer "F.Cu") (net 12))
 (segment (start 131.9022 89.4334) (end 131.9296 89.4334) (width 0.2) (layer "F.Cu") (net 12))
 (segment (start 129.54 90.6506) (end 130.685 90.6506) (width 0.2) (layer "F.Cu") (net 12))
 (segment (start 133.4285 89.3166) (end 133.3117 89.4334) (width 0.2) (layer "F.Cu") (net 12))
 (segment (start 130.685 90.6506) (end 131.9022 89.4334) (width 0.2) (layer "F.Cu") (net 12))
 (segment (start 131.9296 88.4936) (end 131.955 88.4682) (width 0.2) (layer "F.Cu") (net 12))
 (segment (start 133.3117 89.4334) (end 131.9296 89.4334) (width 0.2) (layer "F.Cu") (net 12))
 (segment (start 127.0112 91.3638) (end 127.986199 91.3638) (width 0.2) (layer "F.Cu") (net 1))
 (segment (start 128.6002 89.2048) (end 130.3274 87.4776) (width 0.2) (layer "F.Cu") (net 1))
 (segment (start 130.3274 87.4776) (end 130.9604 87.4776) (width 0.2) (layer "F.Cu") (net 1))
 (segment (start 127.986199 91.3638) (end 128.6002 90.749799) (width 0.2) (layer "F.Cu") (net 1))
 (segment (start 128.6002 90.749799) (end 128.6002 89.2048) (width 0.2) (layer "F.Cu") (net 1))
 (segment (start 129.54 91.6706) (end 128.7038 92.5068) (width 0.2) (layer "F.Cu") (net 15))
 (segment (start 126.2634 90.0938) (end 127.0112 90.0938) (width 0.2) (layer "F.Cu") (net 15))
 (segment (start 125.476 90.8812) (end 126.2634 90.0938) (width 0.2) (layer "F.Cu") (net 15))
 (segment (start 125.476 92.075) (end 125.476 90.8812) (width 0.2) (layer "F.Cu") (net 15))
 (segment (start 125.9078 92.5068) (end 125.476 92.075) (width 0.2) (layer "F.Cu") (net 15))
 (segment (start 128.7038 92.5068) (end 125.9078 92.5068) (width 0.2) (layer "F.Cu") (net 15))
 (segment (start 127.0112 88.8238) (end 127.356752 88.8238) (width 0.2) (layer "F.Cu") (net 21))
 (segment (start 129.8906 85.1204) (end 133.1818 85.1204) (width 0.2) (layer "F.Cu") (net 21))
 (segment (start 133.1818 85.1204) (end 134.4568 83.8454) (width 0.2) (layer "F.Cu") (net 21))
 (segment (start 128.6922 86.3188) (end 129.8906 85.1204) (width 0.2) (layer "F.Cu") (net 21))
 (segment (start 128.6922 87.488352) (end 128.6922 86.3188) (width 0.2) (layer "F.Cu") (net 21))
 (segment (start 127.356752 88.8238) (end 128.6922 87.488352) (width 0.2) (layer "F.Cu") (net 21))
 (segment (start 129.2098 80.3148) (end 137.7188 80.3148) (width 0.2) (layer "F.Cu") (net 13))
 (segment (start 122.0612 91.3638) (end 124.4234 93.726) (width 0.2) (layer "F.Cu") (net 13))
 (segment (start 123.8992 90.4006) (end 122.936 91.3638) (width 0.2) (layer "F.Cu") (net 13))
 (segment (start 137.7188 80.3148) (end 140.184599 82.780599) (width 0.2) (layer "F.Cu") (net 13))
 (segment (start 140.184599 89.6366) (end 140.184599 88.3158) (width 0.2) (layer "F.Cu") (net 13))
 (segment (start 141.9974 91.4658) (end 140.692999 91.4658) (width 0.2) (layer "F.Cu") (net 13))
 (segment (start 140.184599 90.9574) (end 140.184599 89.6366) (width 0.2) (layer "F.Cu") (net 13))
 (segment (start 123.8992 85.6488) (end 123.8992 90.4006) (width 0.2) (layer "F.Cu") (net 13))
 (segment (start 126.873 82.6516) (end 129.2098 80.3148) (width 0.2) (layer "F.Cu") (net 13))
 (segment (start 121.6914 84.8868) (end 121.6914 83.2866) (width 0.2) (layer "F.Cu") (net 13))
 (segment (start 121.6914 83.2866) (end 122.3264 82.6516) (width 0.2) (layer "F.Cu") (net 13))
 (segment (start 140.184599 82.780599) (end 140.184599 88.3158) (width 0.2) (layer "F.Cu") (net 13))
 (segment (start 140.184599 92.2274) (end 140.184599 90.9574) (width 0.2) (layer "F.Cu") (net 13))
 (segment (start 123.8992 85.6488) (end 122.4534 85.6488) (width 0.2) (layer "F.Cu") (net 13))
 (segment (start 122.4534 85.6488) (end 121.6914 84.8868) (width 0.2) (layer "F.Cu") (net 13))
 (segment (start 122.3264 82.6516) (end 126.873 82.6516) (width 0.2) (layer "F.Cu") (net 13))
 (segment (start 124.4234 93.726) (end 127.7066 93.726) (width 0.2) (layer "F.Cu") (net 13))
 (segment (start 140.692999 91.4658) (end 140.184599 90.9574) (width 0.2) (layer "F.Cu") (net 13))
 (segment (start 122.936 91.3638) (end 122.0612 91.3638) (width 0.2) (layer "F.Cu") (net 13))
 (segment (start 131.9568 83.8454) (end 129.1356 83.8454) (width 0.2) (layer "F.Cu") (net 4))
 (segment (start 129.1356 83.8454) (end 127.4084 85.5726) (width 0.2) (layer "F.Cu") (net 4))
 (segment (start 135.001 81.8896) (end 129.1336 81.8896) (width 0.2) (layer "F.Cu") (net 20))
 (segment (start 128.0942 82.929) (end 128.0942 83.6168) (width 0.2) (layer "F.Cu") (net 20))
 (segment (start 136.9568 83.8454) (end 135.001 81.8896) (width 0.2) (layer "F.Cu") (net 20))
 (segment (start 129.1336 81.8896) (end 128.0942 82.929) (width 0.2) (layer "F.Cu") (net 20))
 (segment (start 139.164601 92.2274) (end 139.164601 90.9574) (width 0.2) (layer "F.Cu") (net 16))
 (segment (start 139.164601 90.9574) (end 139.164601 89.6366) (width 0.2) (layer "F.Cu") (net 16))
 (segment (start 139.164601 92.708001) (end 139.7 93.2434) (width 0.2) (layer "F.Cu") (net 16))
 (segment (start 144.2974 91.9988) (end 144.2974 91.4658) (width 0.2) (layer "F.Cu") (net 16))
 (segment (start 139.164601 88.3158) (end 139.164601 89.6366) (width 0.2) (layer "F.Cu") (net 16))
 (segment (start 139.7 93.2434) (end 143.0528 93.2434) (width 0.2) (layer "F.Cu") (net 16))
 (segment (start 139.164601 92.2274) (end 139.164601 92.708001) (width 0.2) (layer "F.Cu") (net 16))
 (segment (start 143.0528 93.2434) (end 144.2974 91.9988) (width 0.2) (layer "F.Cu") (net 16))
 (segment (start 144.2974 91.4658) (end 144.2974 85.1658) (width 0.2) (layer "F.Cu") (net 16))
 (segment (start 137.3124 91.1406) (end 135.5652 92.8878) (width 0.2) (layer "F.Cu") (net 22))
 (segment (start 137.3124 89.3404) (end 137.3124 91.1406) (width 0.2) (layer "F.Cu") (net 22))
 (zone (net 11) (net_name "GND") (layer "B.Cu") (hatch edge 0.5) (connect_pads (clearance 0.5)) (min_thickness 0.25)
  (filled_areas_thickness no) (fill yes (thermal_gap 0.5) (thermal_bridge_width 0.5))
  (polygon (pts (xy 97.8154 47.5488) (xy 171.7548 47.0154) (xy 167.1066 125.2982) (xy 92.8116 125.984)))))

